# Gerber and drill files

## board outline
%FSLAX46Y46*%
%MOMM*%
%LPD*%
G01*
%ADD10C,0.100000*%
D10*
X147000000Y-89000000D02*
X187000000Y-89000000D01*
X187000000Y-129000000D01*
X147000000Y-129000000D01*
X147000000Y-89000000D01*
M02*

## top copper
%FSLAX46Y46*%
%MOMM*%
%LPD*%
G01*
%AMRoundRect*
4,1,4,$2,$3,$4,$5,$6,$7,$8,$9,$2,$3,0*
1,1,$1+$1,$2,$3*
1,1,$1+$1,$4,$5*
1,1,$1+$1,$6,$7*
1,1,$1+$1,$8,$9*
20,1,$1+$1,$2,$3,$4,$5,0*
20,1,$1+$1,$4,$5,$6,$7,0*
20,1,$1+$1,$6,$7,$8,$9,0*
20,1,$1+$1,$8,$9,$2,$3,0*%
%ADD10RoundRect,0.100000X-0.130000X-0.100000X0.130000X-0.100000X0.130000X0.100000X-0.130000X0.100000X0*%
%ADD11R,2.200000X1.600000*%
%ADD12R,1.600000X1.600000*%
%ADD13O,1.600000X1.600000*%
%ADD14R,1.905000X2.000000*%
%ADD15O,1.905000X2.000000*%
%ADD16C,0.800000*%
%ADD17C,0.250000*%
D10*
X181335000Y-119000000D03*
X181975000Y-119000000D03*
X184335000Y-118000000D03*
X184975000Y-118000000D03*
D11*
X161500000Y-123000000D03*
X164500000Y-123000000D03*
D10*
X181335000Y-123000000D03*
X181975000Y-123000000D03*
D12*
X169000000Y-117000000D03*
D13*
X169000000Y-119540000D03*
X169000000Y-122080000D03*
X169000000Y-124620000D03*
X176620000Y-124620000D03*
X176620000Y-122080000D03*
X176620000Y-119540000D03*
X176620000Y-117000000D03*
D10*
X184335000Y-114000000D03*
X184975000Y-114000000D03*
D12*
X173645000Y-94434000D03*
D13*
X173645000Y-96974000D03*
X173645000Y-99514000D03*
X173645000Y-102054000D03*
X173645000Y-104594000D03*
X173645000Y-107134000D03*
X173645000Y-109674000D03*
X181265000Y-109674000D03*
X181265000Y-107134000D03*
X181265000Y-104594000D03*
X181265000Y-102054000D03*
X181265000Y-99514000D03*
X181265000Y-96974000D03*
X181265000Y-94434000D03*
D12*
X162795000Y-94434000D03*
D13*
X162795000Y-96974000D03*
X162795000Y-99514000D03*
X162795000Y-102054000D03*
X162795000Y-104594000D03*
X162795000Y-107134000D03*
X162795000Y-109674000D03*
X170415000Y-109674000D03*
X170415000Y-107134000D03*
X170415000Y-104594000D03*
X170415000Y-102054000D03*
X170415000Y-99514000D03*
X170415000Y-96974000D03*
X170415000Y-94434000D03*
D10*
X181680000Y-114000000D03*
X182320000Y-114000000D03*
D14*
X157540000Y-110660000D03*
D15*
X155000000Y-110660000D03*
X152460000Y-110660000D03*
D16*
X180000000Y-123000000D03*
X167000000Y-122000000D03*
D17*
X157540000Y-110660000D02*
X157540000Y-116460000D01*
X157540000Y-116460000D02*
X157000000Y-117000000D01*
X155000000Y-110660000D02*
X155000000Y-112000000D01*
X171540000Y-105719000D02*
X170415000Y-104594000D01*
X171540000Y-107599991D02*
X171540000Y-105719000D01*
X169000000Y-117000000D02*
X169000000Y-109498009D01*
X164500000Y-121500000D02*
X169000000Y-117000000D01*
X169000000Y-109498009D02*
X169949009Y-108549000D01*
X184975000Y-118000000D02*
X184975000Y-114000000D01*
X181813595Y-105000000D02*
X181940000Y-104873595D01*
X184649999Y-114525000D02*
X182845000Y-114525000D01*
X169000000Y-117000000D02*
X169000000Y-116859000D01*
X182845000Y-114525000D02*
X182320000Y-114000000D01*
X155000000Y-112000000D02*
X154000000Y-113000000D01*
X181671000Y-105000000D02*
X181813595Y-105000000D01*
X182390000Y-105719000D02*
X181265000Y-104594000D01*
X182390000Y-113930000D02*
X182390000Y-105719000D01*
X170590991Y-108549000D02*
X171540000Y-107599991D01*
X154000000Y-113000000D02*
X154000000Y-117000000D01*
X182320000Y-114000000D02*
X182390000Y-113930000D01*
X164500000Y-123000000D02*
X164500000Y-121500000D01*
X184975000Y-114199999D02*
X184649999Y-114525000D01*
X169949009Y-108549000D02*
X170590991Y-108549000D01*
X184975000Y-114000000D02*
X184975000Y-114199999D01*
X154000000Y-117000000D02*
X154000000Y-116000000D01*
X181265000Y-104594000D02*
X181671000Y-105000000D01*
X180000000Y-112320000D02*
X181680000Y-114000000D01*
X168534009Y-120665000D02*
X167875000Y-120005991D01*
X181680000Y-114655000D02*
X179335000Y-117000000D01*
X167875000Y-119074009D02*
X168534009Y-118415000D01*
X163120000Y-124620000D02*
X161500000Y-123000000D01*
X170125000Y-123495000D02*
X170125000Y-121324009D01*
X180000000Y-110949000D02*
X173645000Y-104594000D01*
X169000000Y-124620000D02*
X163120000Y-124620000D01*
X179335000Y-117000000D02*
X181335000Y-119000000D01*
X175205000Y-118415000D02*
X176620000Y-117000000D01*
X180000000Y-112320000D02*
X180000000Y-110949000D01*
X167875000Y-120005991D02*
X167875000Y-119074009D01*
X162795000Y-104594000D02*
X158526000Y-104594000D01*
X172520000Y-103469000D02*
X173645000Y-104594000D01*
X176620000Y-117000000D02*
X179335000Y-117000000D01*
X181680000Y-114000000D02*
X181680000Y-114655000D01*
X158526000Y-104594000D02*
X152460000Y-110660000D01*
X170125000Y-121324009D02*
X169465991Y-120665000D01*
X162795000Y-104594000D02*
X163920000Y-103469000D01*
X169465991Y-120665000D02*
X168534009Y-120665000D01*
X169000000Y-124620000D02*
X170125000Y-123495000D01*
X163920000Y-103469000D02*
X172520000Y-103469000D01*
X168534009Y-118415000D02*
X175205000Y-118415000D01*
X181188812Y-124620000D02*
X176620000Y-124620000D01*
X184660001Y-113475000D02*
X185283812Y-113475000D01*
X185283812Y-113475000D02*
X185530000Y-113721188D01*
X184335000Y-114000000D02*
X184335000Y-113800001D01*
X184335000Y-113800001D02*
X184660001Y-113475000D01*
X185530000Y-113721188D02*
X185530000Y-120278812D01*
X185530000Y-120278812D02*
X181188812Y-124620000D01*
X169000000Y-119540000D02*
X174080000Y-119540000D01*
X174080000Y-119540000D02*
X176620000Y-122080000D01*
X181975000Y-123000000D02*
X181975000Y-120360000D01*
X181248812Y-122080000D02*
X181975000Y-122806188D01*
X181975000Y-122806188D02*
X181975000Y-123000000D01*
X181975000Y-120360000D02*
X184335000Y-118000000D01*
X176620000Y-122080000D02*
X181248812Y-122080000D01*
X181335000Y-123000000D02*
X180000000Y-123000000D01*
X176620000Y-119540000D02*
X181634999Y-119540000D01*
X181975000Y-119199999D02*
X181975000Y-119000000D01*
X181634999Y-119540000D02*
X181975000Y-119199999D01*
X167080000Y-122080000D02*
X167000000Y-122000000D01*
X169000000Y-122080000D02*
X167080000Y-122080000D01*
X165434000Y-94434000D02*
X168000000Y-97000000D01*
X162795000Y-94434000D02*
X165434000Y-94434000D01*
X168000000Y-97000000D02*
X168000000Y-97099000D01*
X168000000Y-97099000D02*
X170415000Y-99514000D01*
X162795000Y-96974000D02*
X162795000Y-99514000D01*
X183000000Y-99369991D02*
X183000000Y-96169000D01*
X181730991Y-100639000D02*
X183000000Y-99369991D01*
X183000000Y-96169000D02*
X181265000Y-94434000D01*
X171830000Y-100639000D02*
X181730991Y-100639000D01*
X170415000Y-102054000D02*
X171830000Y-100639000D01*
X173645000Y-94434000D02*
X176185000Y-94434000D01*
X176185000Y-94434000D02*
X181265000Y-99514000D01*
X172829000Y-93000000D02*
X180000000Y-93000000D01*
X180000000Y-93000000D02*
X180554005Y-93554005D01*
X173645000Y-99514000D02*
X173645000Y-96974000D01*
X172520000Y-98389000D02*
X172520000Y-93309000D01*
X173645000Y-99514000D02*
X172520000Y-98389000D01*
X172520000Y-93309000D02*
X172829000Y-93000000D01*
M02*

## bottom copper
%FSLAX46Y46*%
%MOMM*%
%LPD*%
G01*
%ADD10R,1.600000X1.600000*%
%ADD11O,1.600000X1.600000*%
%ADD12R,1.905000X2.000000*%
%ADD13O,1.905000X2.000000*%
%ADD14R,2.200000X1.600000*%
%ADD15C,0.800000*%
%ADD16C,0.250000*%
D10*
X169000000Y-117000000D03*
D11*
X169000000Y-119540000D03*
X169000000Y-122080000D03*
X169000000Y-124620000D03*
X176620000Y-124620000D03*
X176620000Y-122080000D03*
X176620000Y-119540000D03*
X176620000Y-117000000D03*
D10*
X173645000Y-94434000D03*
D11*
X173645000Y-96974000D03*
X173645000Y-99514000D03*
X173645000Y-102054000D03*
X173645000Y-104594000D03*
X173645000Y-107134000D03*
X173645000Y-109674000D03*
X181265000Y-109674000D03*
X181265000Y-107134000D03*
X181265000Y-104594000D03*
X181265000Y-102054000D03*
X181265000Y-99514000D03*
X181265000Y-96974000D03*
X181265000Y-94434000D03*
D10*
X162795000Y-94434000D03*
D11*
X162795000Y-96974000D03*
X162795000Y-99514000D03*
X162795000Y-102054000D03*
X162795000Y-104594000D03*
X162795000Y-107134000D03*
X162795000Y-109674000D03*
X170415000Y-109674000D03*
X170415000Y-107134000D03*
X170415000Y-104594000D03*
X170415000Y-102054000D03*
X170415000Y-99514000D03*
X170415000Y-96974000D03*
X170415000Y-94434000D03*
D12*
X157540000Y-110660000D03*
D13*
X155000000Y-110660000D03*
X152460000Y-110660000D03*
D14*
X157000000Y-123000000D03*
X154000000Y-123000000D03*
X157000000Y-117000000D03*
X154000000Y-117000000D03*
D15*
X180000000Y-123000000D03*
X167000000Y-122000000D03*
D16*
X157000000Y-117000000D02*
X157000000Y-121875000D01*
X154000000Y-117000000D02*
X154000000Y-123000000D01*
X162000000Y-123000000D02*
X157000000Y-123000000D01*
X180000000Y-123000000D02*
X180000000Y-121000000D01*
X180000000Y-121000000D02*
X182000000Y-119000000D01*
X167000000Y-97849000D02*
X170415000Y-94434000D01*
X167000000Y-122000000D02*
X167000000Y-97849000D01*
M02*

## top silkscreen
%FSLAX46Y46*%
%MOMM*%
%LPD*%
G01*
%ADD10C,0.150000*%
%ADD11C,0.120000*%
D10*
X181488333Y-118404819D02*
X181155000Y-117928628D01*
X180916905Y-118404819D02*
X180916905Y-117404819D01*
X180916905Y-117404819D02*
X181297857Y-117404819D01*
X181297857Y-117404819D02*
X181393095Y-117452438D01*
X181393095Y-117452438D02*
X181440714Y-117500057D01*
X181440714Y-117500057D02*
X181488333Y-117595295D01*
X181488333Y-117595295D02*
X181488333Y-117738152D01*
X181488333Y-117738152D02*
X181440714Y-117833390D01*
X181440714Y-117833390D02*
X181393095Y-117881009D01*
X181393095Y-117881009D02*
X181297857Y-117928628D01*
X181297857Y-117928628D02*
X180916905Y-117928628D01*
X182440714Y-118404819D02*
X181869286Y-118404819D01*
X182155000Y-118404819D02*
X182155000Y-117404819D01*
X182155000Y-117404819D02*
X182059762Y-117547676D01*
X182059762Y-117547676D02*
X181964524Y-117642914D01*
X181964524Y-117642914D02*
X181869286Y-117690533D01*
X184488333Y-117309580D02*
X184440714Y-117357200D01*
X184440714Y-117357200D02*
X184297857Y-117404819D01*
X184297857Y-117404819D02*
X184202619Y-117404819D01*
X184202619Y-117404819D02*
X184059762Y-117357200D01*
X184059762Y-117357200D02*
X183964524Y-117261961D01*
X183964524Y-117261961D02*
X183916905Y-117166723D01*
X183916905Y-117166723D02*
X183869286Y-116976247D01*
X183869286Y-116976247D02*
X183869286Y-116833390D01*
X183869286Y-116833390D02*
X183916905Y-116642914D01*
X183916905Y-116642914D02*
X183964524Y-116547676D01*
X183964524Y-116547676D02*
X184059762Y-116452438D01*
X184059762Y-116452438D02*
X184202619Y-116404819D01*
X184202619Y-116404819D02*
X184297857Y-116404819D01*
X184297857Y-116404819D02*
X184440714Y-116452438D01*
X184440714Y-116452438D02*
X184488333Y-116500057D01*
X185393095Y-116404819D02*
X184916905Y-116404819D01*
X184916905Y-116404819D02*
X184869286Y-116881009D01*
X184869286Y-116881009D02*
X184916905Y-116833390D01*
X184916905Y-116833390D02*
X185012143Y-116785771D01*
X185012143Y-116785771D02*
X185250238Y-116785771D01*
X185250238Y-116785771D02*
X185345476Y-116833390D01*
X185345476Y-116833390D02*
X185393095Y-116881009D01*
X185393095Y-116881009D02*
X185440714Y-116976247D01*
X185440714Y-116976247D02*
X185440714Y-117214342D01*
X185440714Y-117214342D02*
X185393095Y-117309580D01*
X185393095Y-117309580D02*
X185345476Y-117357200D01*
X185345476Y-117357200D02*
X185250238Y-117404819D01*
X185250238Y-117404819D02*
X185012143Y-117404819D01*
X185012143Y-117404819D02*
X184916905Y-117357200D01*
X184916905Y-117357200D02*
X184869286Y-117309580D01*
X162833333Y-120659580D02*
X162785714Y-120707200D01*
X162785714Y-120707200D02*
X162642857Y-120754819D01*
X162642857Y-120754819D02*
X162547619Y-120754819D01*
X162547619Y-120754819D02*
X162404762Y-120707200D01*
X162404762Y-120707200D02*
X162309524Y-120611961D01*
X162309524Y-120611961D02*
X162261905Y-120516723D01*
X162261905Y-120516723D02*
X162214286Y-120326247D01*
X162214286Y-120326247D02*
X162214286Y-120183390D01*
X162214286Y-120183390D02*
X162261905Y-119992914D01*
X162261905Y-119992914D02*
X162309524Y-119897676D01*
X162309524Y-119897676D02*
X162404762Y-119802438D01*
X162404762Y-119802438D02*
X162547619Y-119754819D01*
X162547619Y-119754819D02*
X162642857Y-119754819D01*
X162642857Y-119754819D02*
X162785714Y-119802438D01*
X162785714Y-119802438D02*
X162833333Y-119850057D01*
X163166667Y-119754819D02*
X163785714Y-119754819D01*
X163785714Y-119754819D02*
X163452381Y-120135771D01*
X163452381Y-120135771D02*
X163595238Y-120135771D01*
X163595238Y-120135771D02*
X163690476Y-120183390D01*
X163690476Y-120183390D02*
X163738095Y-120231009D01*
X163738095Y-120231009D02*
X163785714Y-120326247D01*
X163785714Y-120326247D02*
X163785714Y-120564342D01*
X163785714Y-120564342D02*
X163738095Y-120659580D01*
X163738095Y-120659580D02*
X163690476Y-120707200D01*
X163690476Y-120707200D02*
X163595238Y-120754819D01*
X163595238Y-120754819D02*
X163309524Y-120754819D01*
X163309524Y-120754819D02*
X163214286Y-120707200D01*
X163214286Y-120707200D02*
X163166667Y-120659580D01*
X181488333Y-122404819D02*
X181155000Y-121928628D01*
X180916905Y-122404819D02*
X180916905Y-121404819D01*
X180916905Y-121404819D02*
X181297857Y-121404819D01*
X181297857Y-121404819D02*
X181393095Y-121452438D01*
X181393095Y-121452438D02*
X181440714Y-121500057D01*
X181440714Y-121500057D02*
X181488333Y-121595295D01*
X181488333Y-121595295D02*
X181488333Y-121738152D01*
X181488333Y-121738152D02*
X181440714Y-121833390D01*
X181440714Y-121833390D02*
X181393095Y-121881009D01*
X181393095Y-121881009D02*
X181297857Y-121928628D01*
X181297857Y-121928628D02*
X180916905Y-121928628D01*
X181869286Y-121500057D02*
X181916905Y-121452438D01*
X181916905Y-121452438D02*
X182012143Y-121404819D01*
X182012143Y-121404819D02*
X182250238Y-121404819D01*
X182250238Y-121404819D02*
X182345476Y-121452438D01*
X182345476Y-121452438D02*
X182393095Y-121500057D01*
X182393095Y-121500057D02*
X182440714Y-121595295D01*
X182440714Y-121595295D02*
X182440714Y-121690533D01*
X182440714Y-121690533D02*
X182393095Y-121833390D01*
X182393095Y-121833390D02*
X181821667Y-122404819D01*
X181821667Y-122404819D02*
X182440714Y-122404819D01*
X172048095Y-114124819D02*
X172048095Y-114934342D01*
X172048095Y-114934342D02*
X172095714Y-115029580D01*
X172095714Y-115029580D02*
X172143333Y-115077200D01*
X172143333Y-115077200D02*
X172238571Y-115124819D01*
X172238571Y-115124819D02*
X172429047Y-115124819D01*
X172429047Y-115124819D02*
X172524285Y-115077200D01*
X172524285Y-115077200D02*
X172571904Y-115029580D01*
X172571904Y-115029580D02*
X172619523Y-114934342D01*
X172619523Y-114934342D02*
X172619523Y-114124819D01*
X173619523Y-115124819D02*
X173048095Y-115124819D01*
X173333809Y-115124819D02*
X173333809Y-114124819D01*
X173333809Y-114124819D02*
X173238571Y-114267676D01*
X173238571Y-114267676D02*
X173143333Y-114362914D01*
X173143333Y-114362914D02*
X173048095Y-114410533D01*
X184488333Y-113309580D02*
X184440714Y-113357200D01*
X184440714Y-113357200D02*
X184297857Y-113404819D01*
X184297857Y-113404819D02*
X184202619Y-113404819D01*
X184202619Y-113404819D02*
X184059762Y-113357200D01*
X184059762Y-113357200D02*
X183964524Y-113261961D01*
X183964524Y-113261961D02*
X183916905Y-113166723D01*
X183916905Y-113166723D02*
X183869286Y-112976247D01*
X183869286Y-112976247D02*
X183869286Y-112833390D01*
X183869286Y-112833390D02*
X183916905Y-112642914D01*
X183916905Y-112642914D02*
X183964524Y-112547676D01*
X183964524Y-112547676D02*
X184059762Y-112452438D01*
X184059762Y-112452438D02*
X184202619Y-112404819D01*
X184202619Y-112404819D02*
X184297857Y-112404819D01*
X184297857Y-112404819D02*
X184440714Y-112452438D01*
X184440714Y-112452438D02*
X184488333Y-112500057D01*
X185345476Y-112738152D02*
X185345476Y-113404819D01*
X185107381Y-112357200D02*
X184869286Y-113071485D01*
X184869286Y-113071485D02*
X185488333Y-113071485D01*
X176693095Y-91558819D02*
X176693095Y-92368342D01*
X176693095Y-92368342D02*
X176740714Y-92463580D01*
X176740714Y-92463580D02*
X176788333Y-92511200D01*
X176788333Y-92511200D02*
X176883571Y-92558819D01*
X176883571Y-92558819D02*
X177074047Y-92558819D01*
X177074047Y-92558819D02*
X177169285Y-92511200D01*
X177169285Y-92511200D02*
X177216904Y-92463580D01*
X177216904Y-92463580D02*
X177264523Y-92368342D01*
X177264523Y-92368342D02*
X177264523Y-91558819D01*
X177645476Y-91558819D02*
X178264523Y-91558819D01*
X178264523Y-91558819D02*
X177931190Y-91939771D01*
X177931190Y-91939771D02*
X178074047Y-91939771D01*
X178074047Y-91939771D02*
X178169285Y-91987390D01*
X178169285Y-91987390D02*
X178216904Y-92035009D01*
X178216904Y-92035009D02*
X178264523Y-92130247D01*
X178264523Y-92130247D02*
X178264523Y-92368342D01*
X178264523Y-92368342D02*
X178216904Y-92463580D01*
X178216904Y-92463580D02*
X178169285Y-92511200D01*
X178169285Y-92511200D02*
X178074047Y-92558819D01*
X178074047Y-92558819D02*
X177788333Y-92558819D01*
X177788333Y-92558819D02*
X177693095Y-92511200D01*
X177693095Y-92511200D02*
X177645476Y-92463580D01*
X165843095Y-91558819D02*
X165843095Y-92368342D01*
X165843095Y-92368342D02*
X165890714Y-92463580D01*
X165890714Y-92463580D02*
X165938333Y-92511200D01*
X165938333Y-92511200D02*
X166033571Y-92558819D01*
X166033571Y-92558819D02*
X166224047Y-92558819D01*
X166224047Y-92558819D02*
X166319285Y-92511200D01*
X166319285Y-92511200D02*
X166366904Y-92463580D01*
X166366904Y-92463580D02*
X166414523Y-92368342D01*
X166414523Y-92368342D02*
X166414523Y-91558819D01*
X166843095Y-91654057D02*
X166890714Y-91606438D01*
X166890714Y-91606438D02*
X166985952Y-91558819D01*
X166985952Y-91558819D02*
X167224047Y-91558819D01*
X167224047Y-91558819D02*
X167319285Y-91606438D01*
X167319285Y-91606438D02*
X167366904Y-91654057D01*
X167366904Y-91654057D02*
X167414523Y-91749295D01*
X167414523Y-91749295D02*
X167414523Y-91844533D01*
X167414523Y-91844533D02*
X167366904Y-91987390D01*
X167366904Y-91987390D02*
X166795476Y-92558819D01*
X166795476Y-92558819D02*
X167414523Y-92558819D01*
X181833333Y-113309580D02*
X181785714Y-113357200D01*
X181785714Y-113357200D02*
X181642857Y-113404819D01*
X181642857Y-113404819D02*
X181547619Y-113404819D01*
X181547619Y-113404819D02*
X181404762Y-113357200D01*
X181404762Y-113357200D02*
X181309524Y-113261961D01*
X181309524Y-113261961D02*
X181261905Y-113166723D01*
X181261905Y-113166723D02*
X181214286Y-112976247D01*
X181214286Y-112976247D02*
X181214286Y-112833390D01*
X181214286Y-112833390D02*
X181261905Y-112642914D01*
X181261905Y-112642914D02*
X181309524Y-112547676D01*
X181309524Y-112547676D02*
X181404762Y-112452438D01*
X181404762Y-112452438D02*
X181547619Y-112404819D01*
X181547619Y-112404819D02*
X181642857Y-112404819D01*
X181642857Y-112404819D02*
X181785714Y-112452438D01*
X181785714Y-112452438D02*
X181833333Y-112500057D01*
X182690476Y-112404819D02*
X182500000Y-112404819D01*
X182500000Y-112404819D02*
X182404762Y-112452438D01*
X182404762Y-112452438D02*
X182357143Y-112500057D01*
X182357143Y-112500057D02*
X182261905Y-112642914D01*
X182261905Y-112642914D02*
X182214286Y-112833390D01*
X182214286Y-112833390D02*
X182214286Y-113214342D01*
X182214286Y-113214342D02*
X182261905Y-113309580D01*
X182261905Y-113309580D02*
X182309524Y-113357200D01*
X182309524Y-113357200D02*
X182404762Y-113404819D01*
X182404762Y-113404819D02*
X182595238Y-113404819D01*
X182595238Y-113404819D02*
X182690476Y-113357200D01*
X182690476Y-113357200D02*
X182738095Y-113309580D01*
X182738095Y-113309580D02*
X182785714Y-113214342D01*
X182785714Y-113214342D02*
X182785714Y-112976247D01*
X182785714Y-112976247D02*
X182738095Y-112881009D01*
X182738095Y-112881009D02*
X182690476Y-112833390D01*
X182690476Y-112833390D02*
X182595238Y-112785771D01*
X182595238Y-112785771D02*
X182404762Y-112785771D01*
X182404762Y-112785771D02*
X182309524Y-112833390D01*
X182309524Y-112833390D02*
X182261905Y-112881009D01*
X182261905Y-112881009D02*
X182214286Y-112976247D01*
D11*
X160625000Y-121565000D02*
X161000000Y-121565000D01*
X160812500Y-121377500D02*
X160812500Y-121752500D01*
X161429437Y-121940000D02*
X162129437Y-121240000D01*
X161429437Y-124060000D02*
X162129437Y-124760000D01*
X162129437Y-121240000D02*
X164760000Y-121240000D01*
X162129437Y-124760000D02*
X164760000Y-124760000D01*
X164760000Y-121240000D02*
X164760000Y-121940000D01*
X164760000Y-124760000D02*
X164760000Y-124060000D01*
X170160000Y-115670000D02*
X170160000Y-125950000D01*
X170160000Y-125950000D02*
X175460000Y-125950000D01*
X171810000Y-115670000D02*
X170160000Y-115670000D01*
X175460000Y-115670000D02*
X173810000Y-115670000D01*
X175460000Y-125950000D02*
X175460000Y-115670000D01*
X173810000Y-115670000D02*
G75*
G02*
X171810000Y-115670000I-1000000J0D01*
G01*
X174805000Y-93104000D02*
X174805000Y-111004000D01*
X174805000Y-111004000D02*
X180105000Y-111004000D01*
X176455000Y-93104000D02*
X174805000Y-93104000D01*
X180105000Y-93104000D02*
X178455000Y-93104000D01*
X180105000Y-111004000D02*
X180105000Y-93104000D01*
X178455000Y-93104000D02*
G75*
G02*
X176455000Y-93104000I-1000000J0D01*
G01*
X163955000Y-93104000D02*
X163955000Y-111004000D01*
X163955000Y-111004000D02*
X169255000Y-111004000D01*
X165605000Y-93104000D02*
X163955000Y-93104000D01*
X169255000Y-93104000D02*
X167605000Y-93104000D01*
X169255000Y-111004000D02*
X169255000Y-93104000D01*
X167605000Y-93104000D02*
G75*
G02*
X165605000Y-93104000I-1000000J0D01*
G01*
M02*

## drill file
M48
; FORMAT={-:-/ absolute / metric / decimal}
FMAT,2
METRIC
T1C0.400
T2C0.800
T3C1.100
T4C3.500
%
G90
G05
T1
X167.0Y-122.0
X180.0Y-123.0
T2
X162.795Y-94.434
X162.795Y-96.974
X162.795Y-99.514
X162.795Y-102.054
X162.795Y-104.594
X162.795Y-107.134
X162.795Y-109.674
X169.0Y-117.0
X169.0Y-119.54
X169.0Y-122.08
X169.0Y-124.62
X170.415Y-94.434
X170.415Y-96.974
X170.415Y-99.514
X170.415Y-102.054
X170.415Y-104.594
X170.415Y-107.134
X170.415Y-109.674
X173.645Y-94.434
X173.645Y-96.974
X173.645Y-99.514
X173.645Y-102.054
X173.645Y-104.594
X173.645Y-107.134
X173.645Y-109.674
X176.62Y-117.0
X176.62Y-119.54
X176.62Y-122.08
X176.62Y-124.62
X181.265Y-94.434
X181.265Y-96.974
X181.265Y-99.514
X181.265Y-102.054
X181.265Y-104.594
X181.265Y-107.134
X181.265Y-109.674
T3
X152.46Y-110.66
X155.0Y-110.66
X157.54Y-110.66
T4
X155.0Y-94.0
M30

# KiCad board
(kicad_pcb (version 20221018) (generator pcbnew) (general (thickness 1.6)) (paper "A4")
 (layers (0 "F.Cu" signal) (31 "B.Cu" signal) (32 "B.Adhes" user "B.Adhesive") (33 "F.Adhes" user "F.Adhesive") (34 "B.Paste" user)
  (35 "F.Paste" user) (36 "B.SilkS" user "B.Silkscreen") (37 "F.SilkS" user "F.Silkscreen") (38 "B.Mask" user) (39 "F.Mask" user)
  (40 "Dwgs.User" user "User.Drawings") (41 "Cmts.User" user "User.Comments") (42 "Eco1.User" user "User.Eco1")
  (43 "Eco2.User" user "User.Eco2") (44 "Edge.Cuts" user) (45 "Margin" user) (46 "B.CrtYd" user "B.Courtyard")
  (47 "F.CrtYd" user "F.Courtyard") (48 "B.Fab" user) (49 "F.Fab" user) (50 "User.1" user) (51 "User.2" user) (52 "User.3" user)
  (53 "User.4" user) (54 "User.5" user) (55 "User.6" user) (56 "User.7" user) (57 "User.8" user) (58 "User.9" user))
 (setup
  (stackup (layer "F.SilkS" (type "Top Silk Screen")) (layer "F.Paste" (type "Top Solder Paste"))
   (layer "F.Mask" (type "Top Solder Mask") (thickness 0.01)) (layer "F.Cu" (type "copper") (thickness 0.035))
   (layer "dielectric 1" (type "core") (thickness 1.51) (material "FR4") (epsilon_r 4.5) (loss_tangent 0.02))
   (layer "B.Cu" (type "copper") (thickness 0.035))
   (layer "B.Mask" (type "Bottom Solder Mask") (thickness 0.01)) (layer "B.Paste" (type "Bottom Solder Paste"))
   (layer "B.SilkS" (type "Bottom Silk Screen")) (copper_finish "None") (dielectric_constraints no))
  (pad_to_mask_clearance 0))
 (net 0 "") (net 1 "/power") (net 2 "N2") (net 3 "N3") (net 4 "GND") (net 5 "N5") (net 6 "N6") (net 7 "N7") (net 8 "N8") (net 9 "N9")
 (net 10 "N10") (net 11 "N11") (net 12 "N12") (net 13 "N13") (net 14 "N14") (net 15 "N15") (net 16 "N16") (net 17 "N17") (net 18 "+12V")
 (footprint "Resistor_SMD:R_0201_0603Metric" (layer "F.Cu") (at 181.655 119)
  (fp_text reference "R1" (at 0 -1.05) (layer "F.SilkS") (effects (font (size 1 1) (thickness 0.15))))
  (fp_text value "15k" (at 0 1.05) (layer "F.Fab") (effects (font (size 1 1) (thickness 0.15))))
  (pad "" smd roundrect (at -0.345 0) (size 0.318 0.36) (layers "F.Paste") (roundrect_rratio 0.25))
  (pad "" smd roundrect (at 0.345 0) (size 0.318 0.36) (layers "F.Paste") (roundrect_rratio 0.25))
  (pad "1" smd roundrect (at -0.32 0) (size 0.46 0.4) (layers "F.Cu" "F.Mask") (roundrect_rratio 0.25) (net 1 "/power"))
  (pad "2" smd roundrect (at 0.32 0) (size 0.46 0.4) (layers "F.Cu" "F.Mask") (roundrect_rratio 0.25) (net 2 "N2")))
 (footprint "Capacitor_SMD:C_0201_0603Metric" (layer "F.Cu") (at 184.655 118)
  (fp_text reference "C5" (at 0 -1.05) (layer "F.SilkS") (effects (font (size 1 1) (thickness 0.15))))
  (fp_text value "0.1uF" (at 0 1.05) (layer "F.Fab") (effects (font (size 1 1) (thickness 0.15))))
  (pad "" smd roundrect (at -0.345 0) (size 0.318 0.36) (layers "F.Paste") (roundrect_rratio 0.25))
  (pad "" smd roundrect (at 0.345 0) (size 0.318 0.36) (layers "F.Paste") (roundrect_rratio 0.25))
  (pad "1" smd roundrect (at -0.32 0) (size 0.46 0.4) (layers "F.Cu" "F.Mask") (roundrect_rratio 0.25) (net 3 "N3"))
  (pad "2" smd roundrect (at 0.32 0) (size 0.46 0.4) (layers "F.Cu" "F.Mask") (roundrect_rratio 0.25) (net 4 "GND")))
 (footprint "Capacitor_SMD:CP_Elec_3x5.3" (layer "F.Cu") (at 163 123)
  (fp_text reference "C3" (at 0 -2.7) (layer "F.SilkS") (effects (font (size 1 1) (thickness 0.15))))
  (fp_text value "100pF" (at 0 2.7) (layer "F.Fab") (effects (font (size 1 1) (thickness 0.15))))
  (fp_line (start -2.375 -1.435) (end -2 -1.435) (stroke (width 0.12) (type solid)) (layer "F.SilkS"))
  (fp_line (start -2.1875 -1.6225) (end -2.1875 -1.2475) (stroke (width 0.12) (type solid)) (layer "F.SilkS"))
  (fp_line (start -1.570563 -1.06) (end -0.870563 -1.76) (stroke (width 0.12) (type solid)) (layer "F.SilkS"))
  (fp_line (start -1.570563 1.06) (end -0.870563 1.76) (stroke (width 0.12) (type solid)) (layer "F.SilkS"))
  (fp_line (start -0.870563 -1.76) (end 1.76 -1.76) (stroke (width 0.12) (type solid)) (layer "F.SilkS"))
  (fp_line (start -0.870563 1.76) (end 1.76 1.76) (stroke (width 0.12) (type solid)) (layer "F.SilkS"))
  (fp_line (start 1.76 -1.76) (end 1.76 -1.06) (stroke (width 0.12) (type solid)) (layer "F.SilkS"))
  (fp_line (start 1.76 1.76) (end 1.76 1.06) (stroke (width 0.12) (type solid)) (layer "F.SilkS"))
  (pad "1" smd rect (at -1.5 0) (size 2.2 1.6) (layers "F.Cu" "F.Paste" "F.Mask") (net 1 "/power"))
  (pad "2" smd rect (at 1.5 0) (size 2.2 1.6) (layers "F.Cu" "F.Paste" "F.Mask") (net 4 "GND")))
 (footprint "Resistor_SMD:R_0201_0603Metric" (layer "F.Cu") (at 181.655 123)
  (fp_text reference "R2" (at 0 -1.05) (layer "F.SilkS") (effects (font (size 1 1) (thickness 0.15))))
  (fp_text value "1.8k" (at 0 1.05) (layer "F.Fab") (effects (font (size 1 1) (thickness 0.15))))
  (pad "" smd roundrect (at -0.345 0) (size 0.318 0.36) (layers "F.Paste") (roundrect_rratio 0.25))
  (pad "" smd roundrect (at 0.345 0) (size 0.318 0.36) (layers "F.Paste") (roundrect_rratio 0.25))
  (pad "1" smd roundrect (at -0.32 0) (size 0.46 0.4) (layers "F.Cu" "F.Mask") (roundrect_rratio 0.25) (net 2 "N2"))
  (pad "2" smd roundrect (at 0.32 0) (size 0.46 0.4) (layers "F.Cu" "F.Mask") (roundrect_rratio 0.25) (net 3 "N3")))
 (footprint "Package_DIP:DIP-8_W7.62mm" (layer "F.Cu") (at 169 117)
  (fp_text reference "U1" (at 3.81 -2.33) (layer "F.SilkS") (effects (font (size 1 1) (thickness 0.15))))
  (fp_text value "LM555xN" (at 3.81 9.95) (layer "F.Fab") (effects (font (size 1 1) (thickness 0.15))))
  (fp_line (start 1.16 -1.33) (end 1.16 8.95) (stroke (width 0.12) (type solid)) (layer "F.SilkS"))
  (fp_line (start 1.16 8.95) (end 6.46 8.95) (stroke (width 0.12) (type solid)) (layer "F.SilkS"))
  (fp_line (start 2.81 -1.33) (end 1.16 -1.33) (stroke (width 0.12) (type solid)) (layer "F.SilkS"))
  (fp_line (start 6.46 -1.33) (end 4.81 -1.33) (stroke (width 0.12) (type solid)) (layer "F.SilkS"))
  (fp_line (start 6.46 8.95) (end 6.46 -1.33) (stroke (width 0.12) (type solid)) (layer "F.SilkS"))
  (fp_arc (start 4.81 -1.33) (mid 3.81 -0.33) (end 2.81 -1.33) (stroke (width 0.12) (type solid)) (layer "F.SilkS"))
  (pad "1" thru_hole rect (at 0 0) (size 1.6 1.6) (drill 0.8) (layers "*.Cu" "*.Mask") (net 4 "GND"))
  (pad "2" thru_hole oval (at 0 2.54) (size 1.6 1.6) (drill 0.8) (layers "*.Cu" "*.Mask") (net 3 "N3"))
  (pad "3" thru_hole oval (at 0 5.08) (size 1.6 1.6) (drill 0.8) (layers "*.Cu" "*.Mask") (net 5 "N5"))
  (pad "4" thru_hole oval (at 0 7.62) (size 1.6 1.6) (drill 0.8) (layers "*.Cu" "*.Mask") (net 1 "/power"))
  (pad "5" thru_hole oval (at 7.62 7.62) (size 1.6 1.6) (drill 0.8) (layers "*.Cu" "*.Mask") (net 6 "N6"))
  (pad "6" thru_hole oval (at 7.62 5.08) (size 1.6 1.6) (drill 0.8) (layers "*.Cu" "*.Mask") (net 3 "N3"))
  (pad "7" thru_hole oval (at 7.62 2.54) (size 1.6 1.6) (drill 0.8) (layers "*.Cu" "*.Mask") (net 2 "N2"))
  (pad "8" thru_hole oval (at 7.62 0) (size 1.6 1.6) (drill 0.8) (layers "*.Cu" "*.Mask") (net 1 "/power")))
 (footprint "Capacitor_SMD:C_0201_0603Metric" (layer "F.Cu") (at 184.655 114)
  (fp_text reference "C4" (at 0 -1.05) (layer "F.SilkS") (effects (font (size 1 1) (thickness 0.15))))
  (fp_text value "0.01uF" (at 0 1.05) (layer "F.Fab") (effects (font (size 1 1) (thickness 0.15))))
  (pad "" smd roundrect (at -0.345 0) (size 0.318 0.36) (layers "F.Paste") (roundrect_rratio 0.25))
  (pad "" smd roundrect (at 0.345 0) (size 0.318 0.36) (layers "F.Paste") (roundrect_rratio 0.25))
  (pad "1" smd roundrect (at -0.32 0) (size 0.46 0.4) (layers "F.Cu" "F.Mask") (roundrect_rratio 0.25) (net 6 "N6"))
  (pad "2" smd roundrect (at 0.32 0) (size 0.46 0.4) (layers "F.Cu" "F.Mask") (roundrect_rratio 0.25) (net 4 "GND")))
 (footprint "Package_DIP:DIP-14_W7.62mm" (layer "F.Cu") (at 173.645 94.434)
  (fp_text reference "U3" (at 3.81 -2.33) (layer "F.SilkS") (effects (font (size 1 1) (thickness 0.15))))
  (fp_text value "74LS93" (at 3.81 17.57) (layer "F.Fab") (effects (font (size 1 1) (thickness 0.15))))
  (fp_line (start 1.16 -1.33) (end 1.16 16.57) (stroke (width 0.12) (type solid)) (layer "F.SilkS"))
  (fp_line (start 1.16 16.57) (end 6.46 16.57) (stroke (width 0.12) (type solid)) (layer "F.SilkS"))
  (fp_line (start 2.81 -1.33) (end 1.16 -1.33) (stroke (width 0.12) (type solid)) (layer "F.SilkS"))
  (fp_line (start 6.46 -1.33) (end 4.81 -1.33) (stroke (width 0.12) (type solid)) (layer "F.SilkS"))
  (fp_line (start 6.46 16.57) (end 6.46 -1.33) (stroke (width 0.12) (type solid)) (layer "F.SilkS"))
  (fp_arc (start 4.81 -1.33) (mid 3.81 -0.33) (end 2.81 -1.33) (stroke (width 0.12) (type solid)) (layer "F.SilkS"))
  (pad "1" thru_hole rect (at 0 0) (size 1.6 1.6) (drill 0.8) (layers "*.Cu" "*.Mask") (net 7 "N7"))
  (pad "2" thru_hole oval (at 0 2.54) (size 1.6 1.6) (drill 0.8) (layers "*.Cu" "*.Mask") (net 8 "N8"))
  (pad "3" thru_hole oval (at 0 5.08) (size 1.6 1.6) (drill 0.8) (layers "*.Cu" "*.Mask") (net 8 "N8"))
  (pad "4" thru_hole oval (at 0 7.62) (size 1.6 1.6) (drill 0.8) (layers "*.Cu" "*.Mask"))
  (pad "5" thru_hole oval (at 0 10.16) (size 1.6 1.6) (drill 0.8) (layers "*.Cu" "*.Mask") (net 1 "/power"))
  (pad "6" thru_hole oval (at 0 12.7) (size 1.6 1.6) (drill 0.8) (layers "*.Cu" "*.Mask"))
  (pad "7" thru_hole oval (at 0 15.24) (size 1.6 1.6) (drill 0.8) (layers "*.Cu" "*.Mask"))
  (pad "8" thru_hole oval (at 7.62 15.24) (size 1.6 1.6) (drill 0.8) (layers "*.Cu" "*.Mask") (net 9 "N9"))
  (pad "9" thru_hole oval (at 7.62 12.7) (size 1.6 1.6) (drill 0.8) (layers "*.Cu" "*.Mask") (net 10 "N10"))
  (pad "10" thru_hole oval (at 7.62 10.16) (size 1.6 1.6) (drill 0.8) (layers "*.Cu" "*.Mask") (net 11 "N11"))
  (pad "11" thru_hole oval (at 7.62 7.62) (size 1.6 1.6) (drill 0.8) (layers "*.Cu" "*.Mask") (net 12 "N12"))
  (pad "12" thru_hole oval (at 7.62 5.08) (size 1.6 1.6) (drill 0.8) (layers "*.Cu" "*.Mask") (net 7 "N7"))
  (pad "13" thru_hole oval (at 7.62 2.54) (size 1.6 1.6) (drill 0.8) (layers "*.Cu" "*.Mask"))
  (pad "14" thru_hole oval (at 7.62 0) (size 1.6 1.6) (drill 0.8) (layers "*.Cu" "*.Mask") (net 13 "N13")))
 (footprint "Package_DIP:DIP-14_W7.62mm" (layer "F.Cu") (at 162.795 94.434)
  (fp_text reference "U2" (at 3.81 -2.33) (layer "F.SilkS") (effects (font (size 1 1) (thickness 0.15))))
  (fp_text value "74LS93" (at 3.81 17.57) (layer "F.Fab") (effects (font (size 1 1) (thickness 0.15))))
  (fp_line (start 1.16 -1.33) (end 1.16 16.57) (stroke (width 0.12) (type solid)) (layer "F.SilkS"))
  (fp_line (start 1.16 16.57) (end 6.46 16.57) (stroke (width 0.12) (type solid)) (layer "F.SilkS"))
  (fp_line (start 2.81 -1.33) (end 1.16 -1.33) (stroke (width 0.12) (type solid)) (layer "F.SilkS"))
  (fp_line (start 6.46 -1.33) (end 4.81 -1.33) (stroke (width 0.12) (type solid)) (layer "F.SilkS"))
  (fp_line (start 6.46 16.57) (end 6.46 -1.33) (stroke (width 0.12) (type solid)) (layer "F.SilkS"))
  (fp_arc (start 4.81 -1.33) (mid 3.81 -0.33) (end 2.81 -1.33) (stroke (width 0.12) (type solid)) (layer "F.SilkS"))
  (pad "1" thru_hole rect (at 0 0) (size 1.6 1.6) (drill 0.8) (layers "*.Cu" "*.Mask") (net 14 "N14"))
  (pad "2" thru_hole oval (at 0 2.54) (size 1.6 1.6) (drill 0.8) (layers "*.Cu" "*.Mask") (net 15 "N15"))
  (pad "3" thru_hole oval (at 0 5.08) (size 1.6 1.6) (drill 0.8) (layers "*.Cu" "*.Mask") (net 15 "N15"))
  (pad "4" thru_hole oval (at 0 7.62) (size 1.6 1.6) (drill 0.8) (layers "*.Cu" "*.Mask"))
  (pad "5" thru_hole oval (at 0 10.16) (size 1.6 1.6) (drill 0.8) (layers "*.Cu" "*.Mask") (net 1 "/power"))
  (pad "6" thru_hole oval (at 0 12.7) (size 1.6 1.6) (drill 0.8) (layers "*.Cu" "*.Mask"))
  (pad "7" thru_hole oval (at 0 15.24) (size 1.6 1.6) (drill 0.8) (layers "*.Cu" "*.Mask"))
  (pad "8" thru_hole oval (at 7.62 15.24) (size 1.6 1.6) (drill 0.8) (layers "*.Cu" "*.Mask") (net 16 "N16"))
  (pad "9" thru_hole oval (at 7.62 12.7) (size 1.6 1.6) (drill 0.8) (layers "*.Cu" "*.Mask") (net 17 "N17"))
  (pad "10" thru_hole oval (at 7.62 10.16) (size 1.6 1.6) (drill 0.8) (layers "*.Cu" "*.Mask") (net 4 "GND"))
  (pad "11" thru_hole oval (at 7.62 7.62) (size 1.6 1.6) (drill 0.8) (layers "*.Cu" "*.Mask") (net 13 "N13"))
  (pad "12" thru_hole oval (at 7.62 5.08) (size 1.6 1.6) (drill 0.8) (layers "*.Cu" "*.Mask") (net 14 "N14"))
  (pad "13" thru_hole oval (at 7.62 2.54) (size 1.6 1.6) (drill 0.8) (layers "*.Cu" "*.Mask"))
  (pad "14" thru_hole oval (at 7.62 0) (size 1.6 1.6) (drill 0.8) (layers "*.Cu" "*.Mask") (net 5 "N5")))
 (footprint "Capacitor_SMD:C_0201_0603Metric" (layer "F.Cu") (at 182 114)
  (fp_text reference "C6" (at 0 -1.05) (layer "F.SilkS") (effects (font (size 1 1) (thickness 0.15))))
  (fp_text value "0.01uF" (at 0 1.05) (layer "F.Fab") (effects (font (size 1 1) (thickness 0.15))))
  (pad "" smd roundrect (at -0.345 0) (size 0.318 0.36) (layers "F.Paste") (roundrect_rratio 0.25))
  (pad "" smd roundrect (at 0.345 0) (size 0.318 0.36) (layers "F.Paste") (roundrect_rratio 0.25))
  (pad "1" smd roundrect (at -0.32 0) (size 0.46 0.4) (layers "F.Cu" "F.Mask") (roundrect_rratio 0.25) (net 1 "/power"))
  (pad "2" smd roundrect (at 0.32 0) (size 0.46 0.4) (layers "F.Cu" "F.Mask") (roundrect_rratio 0.25) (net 11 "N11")))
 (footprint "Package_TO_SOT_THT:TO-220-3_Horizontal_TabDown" (layer "B.Cu") (at 157.54 110.66 180)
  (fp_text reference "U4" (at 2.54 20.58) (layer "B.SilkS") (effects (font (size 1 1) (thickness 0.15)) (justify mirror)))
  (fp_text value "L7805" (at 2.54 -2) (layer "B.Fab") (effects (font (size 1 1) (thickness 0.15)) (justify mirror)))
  (pad "" np_thru_hole oval (at 2.54 16.66 180) (size 3.5 3.5) (drill 3.5) (layers "*.Cu" "*.Mask"))
  (pad "1" thru_hole rect (at 0 0 180) (size 1.905 2) (drill 1.1) (layers "*.Cu" "*.Mask") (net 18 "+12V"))
  (pad "2" thru_hole oval (at 2.54 0 180) (size 1.905 2) (drill 1.1) (layers "*.Cu" "*.Mask") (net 4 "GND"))
  (pad "3" thru_hole oval (at 5.08 0 180) (size 1.905 2) (drill 1.1) (layers "*.Cu" "*.Mask") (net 1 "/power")))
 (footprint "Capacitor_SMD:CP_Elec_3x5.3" (layer "B.Cu") (at 155.5 123 180)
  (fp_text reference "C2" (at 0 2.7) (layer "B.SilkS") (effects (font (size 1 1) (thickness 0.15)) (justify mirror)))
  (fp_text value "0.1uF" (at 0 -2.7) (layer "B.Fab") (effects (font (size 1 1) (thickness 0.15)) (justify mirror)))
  (pad "1" smd rect (at -1.5 0 180) (size 2.2 1.6) (layers "B.Cu" "B.Paste" "B.Mask") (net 1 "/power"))
  (pad "2" smd rect (at 1.5 0 180) (size 2.2 1.6) (layers "B.Cu" "B.Paste" "B.Mask") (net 4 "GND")))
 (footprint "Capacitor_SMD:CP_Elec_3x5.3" (layer "B.Cu") (at 155.5 117 180)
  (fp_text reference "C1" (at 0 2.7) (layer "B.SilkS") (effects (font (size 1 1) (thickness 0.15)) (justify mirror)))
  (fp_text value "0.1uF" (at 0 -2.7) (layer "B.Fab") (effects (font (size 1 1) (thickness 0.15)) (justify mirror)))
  (pad "1" smd rect (at -1.5 0 180) (size 2.2 1.6) (layers "B.Cu" "B.Paste" "B.Mask") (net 18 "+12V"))
  (pad "2" smd rect (at 1.5 0 180) (size 2.2 1.6) (layers "B.Cu" "B.Paste" "B.Mask") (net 4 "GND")))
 (gr_rect (start 147 89) (end 187 129) (stroke (width 0.1) (type default)) (fill none) (layer "Edge.Cuts"))
 (segment (start 157.54 110.66) (end 157.54 116.46) (width 0.25) (layer "F.Cu") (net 18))
 (segment (start 157.54 116.46) (end 157 117) (width 0.25) (layer "F.Cu") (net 18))
 (segment (start 157 117) (end 157 121.875) (width 0.25) (layer "B.Cu") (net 18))
 (segment (start 155 110.66) (end 155 112) (width 0.25) (layer "F.Cu") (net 4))
 (segment (start 171.54 105.719) (end 170.415 104.594) (width 0.25) (layer "F.Cu") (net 4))
 (segment (start 171.54 107.599991) (end 171.54 105.719) (width 0.25) (layer "F.Cu") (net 4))
 (segment (start 169 117) (end 169 109.498009) (width 0.25) (layer "F.Cu") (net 4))
 (segment (start 164.5 121.5) (end 169 117) (width 0.25) (layer "F.Cu") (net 4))
 (segment (start 169 109.498009) (end 169.949009 108.549) (width 0.25) (layer "F.Cu") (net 4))
 (segment (start 184.975 118) (end 184.975 114) (width 0.25) (layer "F.Cu") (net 4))
 (segment (start 181.813595 105) (end 181.94 104.873595) (width 0.25) (layer "F.Cu") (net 4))
 (segment (start 184.649999 114.525) (end 182.845 114.525) (width 0.25) (layer "F.Cu") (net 4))
 (segment (start 169 117) (end 169 116.859) (width 0.25) (layer "F.Cu") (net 4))
 (segment (start 182.845 114.525) (end 182.32 114) (width 0.25) (layer "F.Cu") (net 4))
 (segment (start 155 112) (end 154 113) (width 0.25) (layer "F.Cu") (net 4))
 (segment (start 181.671 105) (end 181.813595 105) (width 0.25) (layer "F.Cu") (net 4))
 (segment (start 182.39 105.719) (end 181.265 104.594) (width 0.25) (layer "F.Cu") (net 4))
 (segment (start 182.39 113.93) (end 182.39 105.719) (width 0.25) (layer "F.Cu") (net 4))
 (segment (start 170.590991 108.549) (end 171.54 107.599991) (width 0.25) (layer "F.Cu") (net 4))
 (segment (start 154 113) (end 154 117) (width 0.25) (layer "F.Cu") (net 4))
 (segment (start 182.32 114) (end 182.39 113.93) (width 0.25) (layer "F.Cu") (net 4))
 (segment (start 164.5 123) (end 164.5 121.5) (width 0.25) (layer "F.Cu") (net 4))
 (segment (start 184.975 114.199999) (end 184.649999 114.525) (width 0.25) (layer "F.Cu") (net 4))
 (segment (start 169.949009 108.549) (end 170.590991 108.549) (width 0.25) (layer "F.Cu") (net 4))
 (segment (start 184.975 114) (end 184.975 114.199999) (width 0.25) (layer "F.Cu") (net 4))
 (segment (start 154 117) (end 154 116) (width 0.25) (layer "F.Cu") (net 4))
 (segment (start 181.265 104.594) (end 181.671 105) (width 0.25) (layer "F.Cu") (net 4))
 (segment (start 154 117) (end 154 123) (width 0.25) (layer "B.Cu") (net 4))
 (segment (start 180 112.32) (end 181.68 114) (width 0.25) (layer "F.Cu") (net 1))
 (segment (start 168.534009 120.665) (end 167.875 120.005991) (width 0.25) (layer "F.Cu") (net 1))
 (segment (start 181.68 114.655) (end 179.335 117) (width 0.25) (layer "F.Cu") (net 1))
 (segment (start 167.875 119.074009) (end 168.534009 118.415) (width 0.25) (layer "F.Cu") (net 1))
 (segment (start 163.12 124.62) (end 161.5 123) (width 0.25) (layer "F.Cu") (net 1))
 (segment (start 170.125 123.495) (end 170.125 121.324009) (width 0.25) (layer "F.Cu") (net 1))
 (segment (start 180 110.949) (end 173.645 104.594) (width 0.25) (layer "F.Cu") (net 1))
 (segment (start 169 124.62) (end 163.12 124.62) (width 0.25) (layer "F.Cu") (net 1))
 (segment (start 179.335 117) (end 181.335 119) (width 0.25) (layer "F.Cu") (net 1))
 (segment (start 175.205 118.415) (end 176.62 117) (width 0.25) (layer "F.Cu") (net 1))
 (segment (start 180 112.32) (end 180 110.949) (width 0.25) (layer "F.Cu") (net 1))
 (segment (start 167.875 120.005991) (end 167.875 119.074009) (width 0.25) (layer "F.Cu") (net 1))
 (segment (start 162.795 104.594) (end 158.526 104.594) (width 0.25) (layer "F.Cu") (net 1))
 (segment (start 172.52 103.469) (end 173.645 104.594) (width 0.25) (layer "F.Cu") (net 1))
 (segment (start 176.62 117) (end 179.335 117) (width 0.25) (layer "F.Cu") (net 1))
 (segment (start 181.68 114) (end 181.68 114.655) (width 0.25) (layer "F.Cu") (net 1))
 (segment (start 158.526 104.594) (end 152.46 110.66) (width 0.25) (layer "F.Cu") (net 1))
 (segment (start 170.125 121.324009) (end 169.465991 120.665) (width 0.25) (layer "F.Cu") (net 1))
 (segment (start 162.795 104.594) (end 163.92 103.469) (width 0.25) (layer "F.Cu") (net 1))
 (segment (start 169.465991 120.665) (end 168.534009 120.665) (width 0.25) (layer "F.Cu") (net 1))
 (segment (start 169 124.62) (end 170.125 123.495) (width 0.25) (layer "F.Cu") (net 1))
 (segment (start 163.92 103.469) (end 172.52 103.469) (width 0.25) (layer "F.Cu") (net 1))
 (segment (start 168.534009 118.415) (end 175.205 118.415) (width 0.25) (layer "F.Cu") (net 1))
 (segment (start 162 123) (end 157 123) (width 0.25) (layer "B.Cu") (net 1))
 (segment (start 181.188812 124.62) (end 176.62 124.62) (width 0.25) (layer "F.Cu") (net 6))
 (segment (start 184.660001 113.475) (end 185.283812 113.475) (width 0.25) (layer "F.Cu") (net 6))
 (segment (start 185.283812 113.475) (end 185.53 113.721188) (width 0.25) (layer "F.Cu") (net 6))
 (segment (start 184.335 114) (end 184.335 113.800001) (width 0.25) (layer "F.Cu") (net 6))
 (segment (start 184.335 113.800001) (end 184.660001 113.475) (width 0.25) (layer "F.Cu") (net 6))
 (segment (start 185.53 113.721188) (end 185.53 120.278812) (width 0.25) (layer "F.Cu") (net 6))
 (segment (start 185.53 120.278812) (end 181.188812 124.62) (width 0.25) (layer "F.Cu") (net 6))
 (segment (start 169 119.54) (end 174.08 119.54) (width 0.25) (layer "F.Cu") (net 3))
 (segment (start 174.08 119.54) (end 176.62 122.08) (width 0.25) (layer "F.Cu") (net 3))
 (segment (start 181.975 123) (end 181.975 120.36) (width 0.25) (layer "F.Cu") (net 3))
 (segment (start 181.248812 122.08) (end 181.975 122.806188) (width 0.25) (layer "F.Cu") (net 3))
 (segment (start 181.975 122.806188) (end 181.975 123) (width 0.25) (layer "F.Cu") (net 3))
 (segment (start 181.975 120.36) (end 184.335 118) (width 0.25) (layer "F.Cu") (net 3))
 (segment (start 176.62 122.08) (end 181.248812 122.08) (width 0.25) (layer "F.Cu") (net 3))
 (segment (start 181.335 123) (end 180 123) (width 0.25) (layer "F.Cu") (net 2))
 (segment (start 176.62 119.54) (end 181.634999 119.54) (width 0.25) (layer "F.Cu") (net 2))
 (segment (start 181.975 119.199999) (end 181.975 119) (width 0.25) (layer "F.Cu") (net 2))
 (segment (start 181.634999 119.54) (end 181.975 119.199999) (width 0.25) (layer "F.Cu") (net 2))
 (via (at 180 123) (size 0.8) (drill 0.4) (layers "F.Cu" "B.Cu") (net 2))
 (segment (start 180 123) (end 180 121) (width 0.25) (layer "B.Cu") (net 2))
 (segment (start 180 121) (end 182 119) (width 0.25) (layer "B.Cu") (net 2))
 (segment (start 167.08 122.08) (end 167 122) (width 0.25) (layer "F.Cu") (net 5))
 (segment (start 169 122.08) (end 167.08 122.08) (width 0.25) (layer "F.Cu") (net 5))
 (via (at 167 122) (size 0.8) (drill 0.4) (layers "F.Cu" "B.Cu") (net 5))
 (segment (start 167 97.849) (end 170.415 94.434) (width 0.25) (layer "B.Cu") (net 5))
 (segment (start 167 122) (end 167 97.849) (width 0.25) (layer "B.Cu") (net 5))
 (segment (start 165.434 94.434) (end 168 97) (width 0.25) (layer "F.Cu") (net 14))
 (segment (start 162.795 94.434) (end 165.434 94.434) (width 0.25) (layer "F.Cu") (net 14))
 (segment (start 168 97) (end 168 97.099) (width 0.25) (layer "F.Cu") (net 14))
 (segment (start 168 97.099) (end 170.415 99.514) (width 0.25) (layer "F.Cu") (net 14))
 (segment (start 162.795 96.974) (end 162.795 99.514) (width 0.25) (layer "F.Cu") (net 15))
 (segment (start 183 99.369991) (end 183 96.169) (width 0.25) (layer "F.Cu") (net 13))
 (segment (start 181.730991 100.639) (end 183 99.369991) (width 0.25) (layer "F.Cu") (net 13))
 (segment (start 183 96.169) (end 181.265 94.434) (width 0.25) (layer "F.Cu") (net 13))
 (segment (start 171.83 100.639) (end 181.730991 100.639) (width 0.25) (layer "F.Cu") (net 13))
 (segment (start 170.415 102.054) (end 171.83 100.639) (width 0.25) (layer "F.Cu") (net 13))
 (segment (start 173.645 94.434) (end 176.185 94.434) (width 0.25) (layer "F.Cu") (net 7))
 (segment (start 176.185 94.434) (end 181.265 99.514) (width 0.25) (layer "F.Cu") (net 7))
 (segment (start 172.829 93) (end 180 93) (width 0.25) (layer "F.Cu") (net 8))
 (segment (start 180 93) (end 180.554005 93.554005) (width 0.25) (layer "F.Cu") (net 8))
 (segment (start 173.645 99.514) (end 173.645 96.974) (width 0.25) (layer "F.Cu") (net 8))
 (segment (start 172.52 98.389) (end 172.52 93.309) (width 0.25) (layer "F.Cu") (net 8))
 (segment (start 173.645 99.514) (end 172.52 98.389) (width 0.25) (layer "F.Cu") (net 8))
 (segment (start 172.52 93.309) (end 172.829 93) (width 0.25) (layer "F.Cu") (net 8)))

